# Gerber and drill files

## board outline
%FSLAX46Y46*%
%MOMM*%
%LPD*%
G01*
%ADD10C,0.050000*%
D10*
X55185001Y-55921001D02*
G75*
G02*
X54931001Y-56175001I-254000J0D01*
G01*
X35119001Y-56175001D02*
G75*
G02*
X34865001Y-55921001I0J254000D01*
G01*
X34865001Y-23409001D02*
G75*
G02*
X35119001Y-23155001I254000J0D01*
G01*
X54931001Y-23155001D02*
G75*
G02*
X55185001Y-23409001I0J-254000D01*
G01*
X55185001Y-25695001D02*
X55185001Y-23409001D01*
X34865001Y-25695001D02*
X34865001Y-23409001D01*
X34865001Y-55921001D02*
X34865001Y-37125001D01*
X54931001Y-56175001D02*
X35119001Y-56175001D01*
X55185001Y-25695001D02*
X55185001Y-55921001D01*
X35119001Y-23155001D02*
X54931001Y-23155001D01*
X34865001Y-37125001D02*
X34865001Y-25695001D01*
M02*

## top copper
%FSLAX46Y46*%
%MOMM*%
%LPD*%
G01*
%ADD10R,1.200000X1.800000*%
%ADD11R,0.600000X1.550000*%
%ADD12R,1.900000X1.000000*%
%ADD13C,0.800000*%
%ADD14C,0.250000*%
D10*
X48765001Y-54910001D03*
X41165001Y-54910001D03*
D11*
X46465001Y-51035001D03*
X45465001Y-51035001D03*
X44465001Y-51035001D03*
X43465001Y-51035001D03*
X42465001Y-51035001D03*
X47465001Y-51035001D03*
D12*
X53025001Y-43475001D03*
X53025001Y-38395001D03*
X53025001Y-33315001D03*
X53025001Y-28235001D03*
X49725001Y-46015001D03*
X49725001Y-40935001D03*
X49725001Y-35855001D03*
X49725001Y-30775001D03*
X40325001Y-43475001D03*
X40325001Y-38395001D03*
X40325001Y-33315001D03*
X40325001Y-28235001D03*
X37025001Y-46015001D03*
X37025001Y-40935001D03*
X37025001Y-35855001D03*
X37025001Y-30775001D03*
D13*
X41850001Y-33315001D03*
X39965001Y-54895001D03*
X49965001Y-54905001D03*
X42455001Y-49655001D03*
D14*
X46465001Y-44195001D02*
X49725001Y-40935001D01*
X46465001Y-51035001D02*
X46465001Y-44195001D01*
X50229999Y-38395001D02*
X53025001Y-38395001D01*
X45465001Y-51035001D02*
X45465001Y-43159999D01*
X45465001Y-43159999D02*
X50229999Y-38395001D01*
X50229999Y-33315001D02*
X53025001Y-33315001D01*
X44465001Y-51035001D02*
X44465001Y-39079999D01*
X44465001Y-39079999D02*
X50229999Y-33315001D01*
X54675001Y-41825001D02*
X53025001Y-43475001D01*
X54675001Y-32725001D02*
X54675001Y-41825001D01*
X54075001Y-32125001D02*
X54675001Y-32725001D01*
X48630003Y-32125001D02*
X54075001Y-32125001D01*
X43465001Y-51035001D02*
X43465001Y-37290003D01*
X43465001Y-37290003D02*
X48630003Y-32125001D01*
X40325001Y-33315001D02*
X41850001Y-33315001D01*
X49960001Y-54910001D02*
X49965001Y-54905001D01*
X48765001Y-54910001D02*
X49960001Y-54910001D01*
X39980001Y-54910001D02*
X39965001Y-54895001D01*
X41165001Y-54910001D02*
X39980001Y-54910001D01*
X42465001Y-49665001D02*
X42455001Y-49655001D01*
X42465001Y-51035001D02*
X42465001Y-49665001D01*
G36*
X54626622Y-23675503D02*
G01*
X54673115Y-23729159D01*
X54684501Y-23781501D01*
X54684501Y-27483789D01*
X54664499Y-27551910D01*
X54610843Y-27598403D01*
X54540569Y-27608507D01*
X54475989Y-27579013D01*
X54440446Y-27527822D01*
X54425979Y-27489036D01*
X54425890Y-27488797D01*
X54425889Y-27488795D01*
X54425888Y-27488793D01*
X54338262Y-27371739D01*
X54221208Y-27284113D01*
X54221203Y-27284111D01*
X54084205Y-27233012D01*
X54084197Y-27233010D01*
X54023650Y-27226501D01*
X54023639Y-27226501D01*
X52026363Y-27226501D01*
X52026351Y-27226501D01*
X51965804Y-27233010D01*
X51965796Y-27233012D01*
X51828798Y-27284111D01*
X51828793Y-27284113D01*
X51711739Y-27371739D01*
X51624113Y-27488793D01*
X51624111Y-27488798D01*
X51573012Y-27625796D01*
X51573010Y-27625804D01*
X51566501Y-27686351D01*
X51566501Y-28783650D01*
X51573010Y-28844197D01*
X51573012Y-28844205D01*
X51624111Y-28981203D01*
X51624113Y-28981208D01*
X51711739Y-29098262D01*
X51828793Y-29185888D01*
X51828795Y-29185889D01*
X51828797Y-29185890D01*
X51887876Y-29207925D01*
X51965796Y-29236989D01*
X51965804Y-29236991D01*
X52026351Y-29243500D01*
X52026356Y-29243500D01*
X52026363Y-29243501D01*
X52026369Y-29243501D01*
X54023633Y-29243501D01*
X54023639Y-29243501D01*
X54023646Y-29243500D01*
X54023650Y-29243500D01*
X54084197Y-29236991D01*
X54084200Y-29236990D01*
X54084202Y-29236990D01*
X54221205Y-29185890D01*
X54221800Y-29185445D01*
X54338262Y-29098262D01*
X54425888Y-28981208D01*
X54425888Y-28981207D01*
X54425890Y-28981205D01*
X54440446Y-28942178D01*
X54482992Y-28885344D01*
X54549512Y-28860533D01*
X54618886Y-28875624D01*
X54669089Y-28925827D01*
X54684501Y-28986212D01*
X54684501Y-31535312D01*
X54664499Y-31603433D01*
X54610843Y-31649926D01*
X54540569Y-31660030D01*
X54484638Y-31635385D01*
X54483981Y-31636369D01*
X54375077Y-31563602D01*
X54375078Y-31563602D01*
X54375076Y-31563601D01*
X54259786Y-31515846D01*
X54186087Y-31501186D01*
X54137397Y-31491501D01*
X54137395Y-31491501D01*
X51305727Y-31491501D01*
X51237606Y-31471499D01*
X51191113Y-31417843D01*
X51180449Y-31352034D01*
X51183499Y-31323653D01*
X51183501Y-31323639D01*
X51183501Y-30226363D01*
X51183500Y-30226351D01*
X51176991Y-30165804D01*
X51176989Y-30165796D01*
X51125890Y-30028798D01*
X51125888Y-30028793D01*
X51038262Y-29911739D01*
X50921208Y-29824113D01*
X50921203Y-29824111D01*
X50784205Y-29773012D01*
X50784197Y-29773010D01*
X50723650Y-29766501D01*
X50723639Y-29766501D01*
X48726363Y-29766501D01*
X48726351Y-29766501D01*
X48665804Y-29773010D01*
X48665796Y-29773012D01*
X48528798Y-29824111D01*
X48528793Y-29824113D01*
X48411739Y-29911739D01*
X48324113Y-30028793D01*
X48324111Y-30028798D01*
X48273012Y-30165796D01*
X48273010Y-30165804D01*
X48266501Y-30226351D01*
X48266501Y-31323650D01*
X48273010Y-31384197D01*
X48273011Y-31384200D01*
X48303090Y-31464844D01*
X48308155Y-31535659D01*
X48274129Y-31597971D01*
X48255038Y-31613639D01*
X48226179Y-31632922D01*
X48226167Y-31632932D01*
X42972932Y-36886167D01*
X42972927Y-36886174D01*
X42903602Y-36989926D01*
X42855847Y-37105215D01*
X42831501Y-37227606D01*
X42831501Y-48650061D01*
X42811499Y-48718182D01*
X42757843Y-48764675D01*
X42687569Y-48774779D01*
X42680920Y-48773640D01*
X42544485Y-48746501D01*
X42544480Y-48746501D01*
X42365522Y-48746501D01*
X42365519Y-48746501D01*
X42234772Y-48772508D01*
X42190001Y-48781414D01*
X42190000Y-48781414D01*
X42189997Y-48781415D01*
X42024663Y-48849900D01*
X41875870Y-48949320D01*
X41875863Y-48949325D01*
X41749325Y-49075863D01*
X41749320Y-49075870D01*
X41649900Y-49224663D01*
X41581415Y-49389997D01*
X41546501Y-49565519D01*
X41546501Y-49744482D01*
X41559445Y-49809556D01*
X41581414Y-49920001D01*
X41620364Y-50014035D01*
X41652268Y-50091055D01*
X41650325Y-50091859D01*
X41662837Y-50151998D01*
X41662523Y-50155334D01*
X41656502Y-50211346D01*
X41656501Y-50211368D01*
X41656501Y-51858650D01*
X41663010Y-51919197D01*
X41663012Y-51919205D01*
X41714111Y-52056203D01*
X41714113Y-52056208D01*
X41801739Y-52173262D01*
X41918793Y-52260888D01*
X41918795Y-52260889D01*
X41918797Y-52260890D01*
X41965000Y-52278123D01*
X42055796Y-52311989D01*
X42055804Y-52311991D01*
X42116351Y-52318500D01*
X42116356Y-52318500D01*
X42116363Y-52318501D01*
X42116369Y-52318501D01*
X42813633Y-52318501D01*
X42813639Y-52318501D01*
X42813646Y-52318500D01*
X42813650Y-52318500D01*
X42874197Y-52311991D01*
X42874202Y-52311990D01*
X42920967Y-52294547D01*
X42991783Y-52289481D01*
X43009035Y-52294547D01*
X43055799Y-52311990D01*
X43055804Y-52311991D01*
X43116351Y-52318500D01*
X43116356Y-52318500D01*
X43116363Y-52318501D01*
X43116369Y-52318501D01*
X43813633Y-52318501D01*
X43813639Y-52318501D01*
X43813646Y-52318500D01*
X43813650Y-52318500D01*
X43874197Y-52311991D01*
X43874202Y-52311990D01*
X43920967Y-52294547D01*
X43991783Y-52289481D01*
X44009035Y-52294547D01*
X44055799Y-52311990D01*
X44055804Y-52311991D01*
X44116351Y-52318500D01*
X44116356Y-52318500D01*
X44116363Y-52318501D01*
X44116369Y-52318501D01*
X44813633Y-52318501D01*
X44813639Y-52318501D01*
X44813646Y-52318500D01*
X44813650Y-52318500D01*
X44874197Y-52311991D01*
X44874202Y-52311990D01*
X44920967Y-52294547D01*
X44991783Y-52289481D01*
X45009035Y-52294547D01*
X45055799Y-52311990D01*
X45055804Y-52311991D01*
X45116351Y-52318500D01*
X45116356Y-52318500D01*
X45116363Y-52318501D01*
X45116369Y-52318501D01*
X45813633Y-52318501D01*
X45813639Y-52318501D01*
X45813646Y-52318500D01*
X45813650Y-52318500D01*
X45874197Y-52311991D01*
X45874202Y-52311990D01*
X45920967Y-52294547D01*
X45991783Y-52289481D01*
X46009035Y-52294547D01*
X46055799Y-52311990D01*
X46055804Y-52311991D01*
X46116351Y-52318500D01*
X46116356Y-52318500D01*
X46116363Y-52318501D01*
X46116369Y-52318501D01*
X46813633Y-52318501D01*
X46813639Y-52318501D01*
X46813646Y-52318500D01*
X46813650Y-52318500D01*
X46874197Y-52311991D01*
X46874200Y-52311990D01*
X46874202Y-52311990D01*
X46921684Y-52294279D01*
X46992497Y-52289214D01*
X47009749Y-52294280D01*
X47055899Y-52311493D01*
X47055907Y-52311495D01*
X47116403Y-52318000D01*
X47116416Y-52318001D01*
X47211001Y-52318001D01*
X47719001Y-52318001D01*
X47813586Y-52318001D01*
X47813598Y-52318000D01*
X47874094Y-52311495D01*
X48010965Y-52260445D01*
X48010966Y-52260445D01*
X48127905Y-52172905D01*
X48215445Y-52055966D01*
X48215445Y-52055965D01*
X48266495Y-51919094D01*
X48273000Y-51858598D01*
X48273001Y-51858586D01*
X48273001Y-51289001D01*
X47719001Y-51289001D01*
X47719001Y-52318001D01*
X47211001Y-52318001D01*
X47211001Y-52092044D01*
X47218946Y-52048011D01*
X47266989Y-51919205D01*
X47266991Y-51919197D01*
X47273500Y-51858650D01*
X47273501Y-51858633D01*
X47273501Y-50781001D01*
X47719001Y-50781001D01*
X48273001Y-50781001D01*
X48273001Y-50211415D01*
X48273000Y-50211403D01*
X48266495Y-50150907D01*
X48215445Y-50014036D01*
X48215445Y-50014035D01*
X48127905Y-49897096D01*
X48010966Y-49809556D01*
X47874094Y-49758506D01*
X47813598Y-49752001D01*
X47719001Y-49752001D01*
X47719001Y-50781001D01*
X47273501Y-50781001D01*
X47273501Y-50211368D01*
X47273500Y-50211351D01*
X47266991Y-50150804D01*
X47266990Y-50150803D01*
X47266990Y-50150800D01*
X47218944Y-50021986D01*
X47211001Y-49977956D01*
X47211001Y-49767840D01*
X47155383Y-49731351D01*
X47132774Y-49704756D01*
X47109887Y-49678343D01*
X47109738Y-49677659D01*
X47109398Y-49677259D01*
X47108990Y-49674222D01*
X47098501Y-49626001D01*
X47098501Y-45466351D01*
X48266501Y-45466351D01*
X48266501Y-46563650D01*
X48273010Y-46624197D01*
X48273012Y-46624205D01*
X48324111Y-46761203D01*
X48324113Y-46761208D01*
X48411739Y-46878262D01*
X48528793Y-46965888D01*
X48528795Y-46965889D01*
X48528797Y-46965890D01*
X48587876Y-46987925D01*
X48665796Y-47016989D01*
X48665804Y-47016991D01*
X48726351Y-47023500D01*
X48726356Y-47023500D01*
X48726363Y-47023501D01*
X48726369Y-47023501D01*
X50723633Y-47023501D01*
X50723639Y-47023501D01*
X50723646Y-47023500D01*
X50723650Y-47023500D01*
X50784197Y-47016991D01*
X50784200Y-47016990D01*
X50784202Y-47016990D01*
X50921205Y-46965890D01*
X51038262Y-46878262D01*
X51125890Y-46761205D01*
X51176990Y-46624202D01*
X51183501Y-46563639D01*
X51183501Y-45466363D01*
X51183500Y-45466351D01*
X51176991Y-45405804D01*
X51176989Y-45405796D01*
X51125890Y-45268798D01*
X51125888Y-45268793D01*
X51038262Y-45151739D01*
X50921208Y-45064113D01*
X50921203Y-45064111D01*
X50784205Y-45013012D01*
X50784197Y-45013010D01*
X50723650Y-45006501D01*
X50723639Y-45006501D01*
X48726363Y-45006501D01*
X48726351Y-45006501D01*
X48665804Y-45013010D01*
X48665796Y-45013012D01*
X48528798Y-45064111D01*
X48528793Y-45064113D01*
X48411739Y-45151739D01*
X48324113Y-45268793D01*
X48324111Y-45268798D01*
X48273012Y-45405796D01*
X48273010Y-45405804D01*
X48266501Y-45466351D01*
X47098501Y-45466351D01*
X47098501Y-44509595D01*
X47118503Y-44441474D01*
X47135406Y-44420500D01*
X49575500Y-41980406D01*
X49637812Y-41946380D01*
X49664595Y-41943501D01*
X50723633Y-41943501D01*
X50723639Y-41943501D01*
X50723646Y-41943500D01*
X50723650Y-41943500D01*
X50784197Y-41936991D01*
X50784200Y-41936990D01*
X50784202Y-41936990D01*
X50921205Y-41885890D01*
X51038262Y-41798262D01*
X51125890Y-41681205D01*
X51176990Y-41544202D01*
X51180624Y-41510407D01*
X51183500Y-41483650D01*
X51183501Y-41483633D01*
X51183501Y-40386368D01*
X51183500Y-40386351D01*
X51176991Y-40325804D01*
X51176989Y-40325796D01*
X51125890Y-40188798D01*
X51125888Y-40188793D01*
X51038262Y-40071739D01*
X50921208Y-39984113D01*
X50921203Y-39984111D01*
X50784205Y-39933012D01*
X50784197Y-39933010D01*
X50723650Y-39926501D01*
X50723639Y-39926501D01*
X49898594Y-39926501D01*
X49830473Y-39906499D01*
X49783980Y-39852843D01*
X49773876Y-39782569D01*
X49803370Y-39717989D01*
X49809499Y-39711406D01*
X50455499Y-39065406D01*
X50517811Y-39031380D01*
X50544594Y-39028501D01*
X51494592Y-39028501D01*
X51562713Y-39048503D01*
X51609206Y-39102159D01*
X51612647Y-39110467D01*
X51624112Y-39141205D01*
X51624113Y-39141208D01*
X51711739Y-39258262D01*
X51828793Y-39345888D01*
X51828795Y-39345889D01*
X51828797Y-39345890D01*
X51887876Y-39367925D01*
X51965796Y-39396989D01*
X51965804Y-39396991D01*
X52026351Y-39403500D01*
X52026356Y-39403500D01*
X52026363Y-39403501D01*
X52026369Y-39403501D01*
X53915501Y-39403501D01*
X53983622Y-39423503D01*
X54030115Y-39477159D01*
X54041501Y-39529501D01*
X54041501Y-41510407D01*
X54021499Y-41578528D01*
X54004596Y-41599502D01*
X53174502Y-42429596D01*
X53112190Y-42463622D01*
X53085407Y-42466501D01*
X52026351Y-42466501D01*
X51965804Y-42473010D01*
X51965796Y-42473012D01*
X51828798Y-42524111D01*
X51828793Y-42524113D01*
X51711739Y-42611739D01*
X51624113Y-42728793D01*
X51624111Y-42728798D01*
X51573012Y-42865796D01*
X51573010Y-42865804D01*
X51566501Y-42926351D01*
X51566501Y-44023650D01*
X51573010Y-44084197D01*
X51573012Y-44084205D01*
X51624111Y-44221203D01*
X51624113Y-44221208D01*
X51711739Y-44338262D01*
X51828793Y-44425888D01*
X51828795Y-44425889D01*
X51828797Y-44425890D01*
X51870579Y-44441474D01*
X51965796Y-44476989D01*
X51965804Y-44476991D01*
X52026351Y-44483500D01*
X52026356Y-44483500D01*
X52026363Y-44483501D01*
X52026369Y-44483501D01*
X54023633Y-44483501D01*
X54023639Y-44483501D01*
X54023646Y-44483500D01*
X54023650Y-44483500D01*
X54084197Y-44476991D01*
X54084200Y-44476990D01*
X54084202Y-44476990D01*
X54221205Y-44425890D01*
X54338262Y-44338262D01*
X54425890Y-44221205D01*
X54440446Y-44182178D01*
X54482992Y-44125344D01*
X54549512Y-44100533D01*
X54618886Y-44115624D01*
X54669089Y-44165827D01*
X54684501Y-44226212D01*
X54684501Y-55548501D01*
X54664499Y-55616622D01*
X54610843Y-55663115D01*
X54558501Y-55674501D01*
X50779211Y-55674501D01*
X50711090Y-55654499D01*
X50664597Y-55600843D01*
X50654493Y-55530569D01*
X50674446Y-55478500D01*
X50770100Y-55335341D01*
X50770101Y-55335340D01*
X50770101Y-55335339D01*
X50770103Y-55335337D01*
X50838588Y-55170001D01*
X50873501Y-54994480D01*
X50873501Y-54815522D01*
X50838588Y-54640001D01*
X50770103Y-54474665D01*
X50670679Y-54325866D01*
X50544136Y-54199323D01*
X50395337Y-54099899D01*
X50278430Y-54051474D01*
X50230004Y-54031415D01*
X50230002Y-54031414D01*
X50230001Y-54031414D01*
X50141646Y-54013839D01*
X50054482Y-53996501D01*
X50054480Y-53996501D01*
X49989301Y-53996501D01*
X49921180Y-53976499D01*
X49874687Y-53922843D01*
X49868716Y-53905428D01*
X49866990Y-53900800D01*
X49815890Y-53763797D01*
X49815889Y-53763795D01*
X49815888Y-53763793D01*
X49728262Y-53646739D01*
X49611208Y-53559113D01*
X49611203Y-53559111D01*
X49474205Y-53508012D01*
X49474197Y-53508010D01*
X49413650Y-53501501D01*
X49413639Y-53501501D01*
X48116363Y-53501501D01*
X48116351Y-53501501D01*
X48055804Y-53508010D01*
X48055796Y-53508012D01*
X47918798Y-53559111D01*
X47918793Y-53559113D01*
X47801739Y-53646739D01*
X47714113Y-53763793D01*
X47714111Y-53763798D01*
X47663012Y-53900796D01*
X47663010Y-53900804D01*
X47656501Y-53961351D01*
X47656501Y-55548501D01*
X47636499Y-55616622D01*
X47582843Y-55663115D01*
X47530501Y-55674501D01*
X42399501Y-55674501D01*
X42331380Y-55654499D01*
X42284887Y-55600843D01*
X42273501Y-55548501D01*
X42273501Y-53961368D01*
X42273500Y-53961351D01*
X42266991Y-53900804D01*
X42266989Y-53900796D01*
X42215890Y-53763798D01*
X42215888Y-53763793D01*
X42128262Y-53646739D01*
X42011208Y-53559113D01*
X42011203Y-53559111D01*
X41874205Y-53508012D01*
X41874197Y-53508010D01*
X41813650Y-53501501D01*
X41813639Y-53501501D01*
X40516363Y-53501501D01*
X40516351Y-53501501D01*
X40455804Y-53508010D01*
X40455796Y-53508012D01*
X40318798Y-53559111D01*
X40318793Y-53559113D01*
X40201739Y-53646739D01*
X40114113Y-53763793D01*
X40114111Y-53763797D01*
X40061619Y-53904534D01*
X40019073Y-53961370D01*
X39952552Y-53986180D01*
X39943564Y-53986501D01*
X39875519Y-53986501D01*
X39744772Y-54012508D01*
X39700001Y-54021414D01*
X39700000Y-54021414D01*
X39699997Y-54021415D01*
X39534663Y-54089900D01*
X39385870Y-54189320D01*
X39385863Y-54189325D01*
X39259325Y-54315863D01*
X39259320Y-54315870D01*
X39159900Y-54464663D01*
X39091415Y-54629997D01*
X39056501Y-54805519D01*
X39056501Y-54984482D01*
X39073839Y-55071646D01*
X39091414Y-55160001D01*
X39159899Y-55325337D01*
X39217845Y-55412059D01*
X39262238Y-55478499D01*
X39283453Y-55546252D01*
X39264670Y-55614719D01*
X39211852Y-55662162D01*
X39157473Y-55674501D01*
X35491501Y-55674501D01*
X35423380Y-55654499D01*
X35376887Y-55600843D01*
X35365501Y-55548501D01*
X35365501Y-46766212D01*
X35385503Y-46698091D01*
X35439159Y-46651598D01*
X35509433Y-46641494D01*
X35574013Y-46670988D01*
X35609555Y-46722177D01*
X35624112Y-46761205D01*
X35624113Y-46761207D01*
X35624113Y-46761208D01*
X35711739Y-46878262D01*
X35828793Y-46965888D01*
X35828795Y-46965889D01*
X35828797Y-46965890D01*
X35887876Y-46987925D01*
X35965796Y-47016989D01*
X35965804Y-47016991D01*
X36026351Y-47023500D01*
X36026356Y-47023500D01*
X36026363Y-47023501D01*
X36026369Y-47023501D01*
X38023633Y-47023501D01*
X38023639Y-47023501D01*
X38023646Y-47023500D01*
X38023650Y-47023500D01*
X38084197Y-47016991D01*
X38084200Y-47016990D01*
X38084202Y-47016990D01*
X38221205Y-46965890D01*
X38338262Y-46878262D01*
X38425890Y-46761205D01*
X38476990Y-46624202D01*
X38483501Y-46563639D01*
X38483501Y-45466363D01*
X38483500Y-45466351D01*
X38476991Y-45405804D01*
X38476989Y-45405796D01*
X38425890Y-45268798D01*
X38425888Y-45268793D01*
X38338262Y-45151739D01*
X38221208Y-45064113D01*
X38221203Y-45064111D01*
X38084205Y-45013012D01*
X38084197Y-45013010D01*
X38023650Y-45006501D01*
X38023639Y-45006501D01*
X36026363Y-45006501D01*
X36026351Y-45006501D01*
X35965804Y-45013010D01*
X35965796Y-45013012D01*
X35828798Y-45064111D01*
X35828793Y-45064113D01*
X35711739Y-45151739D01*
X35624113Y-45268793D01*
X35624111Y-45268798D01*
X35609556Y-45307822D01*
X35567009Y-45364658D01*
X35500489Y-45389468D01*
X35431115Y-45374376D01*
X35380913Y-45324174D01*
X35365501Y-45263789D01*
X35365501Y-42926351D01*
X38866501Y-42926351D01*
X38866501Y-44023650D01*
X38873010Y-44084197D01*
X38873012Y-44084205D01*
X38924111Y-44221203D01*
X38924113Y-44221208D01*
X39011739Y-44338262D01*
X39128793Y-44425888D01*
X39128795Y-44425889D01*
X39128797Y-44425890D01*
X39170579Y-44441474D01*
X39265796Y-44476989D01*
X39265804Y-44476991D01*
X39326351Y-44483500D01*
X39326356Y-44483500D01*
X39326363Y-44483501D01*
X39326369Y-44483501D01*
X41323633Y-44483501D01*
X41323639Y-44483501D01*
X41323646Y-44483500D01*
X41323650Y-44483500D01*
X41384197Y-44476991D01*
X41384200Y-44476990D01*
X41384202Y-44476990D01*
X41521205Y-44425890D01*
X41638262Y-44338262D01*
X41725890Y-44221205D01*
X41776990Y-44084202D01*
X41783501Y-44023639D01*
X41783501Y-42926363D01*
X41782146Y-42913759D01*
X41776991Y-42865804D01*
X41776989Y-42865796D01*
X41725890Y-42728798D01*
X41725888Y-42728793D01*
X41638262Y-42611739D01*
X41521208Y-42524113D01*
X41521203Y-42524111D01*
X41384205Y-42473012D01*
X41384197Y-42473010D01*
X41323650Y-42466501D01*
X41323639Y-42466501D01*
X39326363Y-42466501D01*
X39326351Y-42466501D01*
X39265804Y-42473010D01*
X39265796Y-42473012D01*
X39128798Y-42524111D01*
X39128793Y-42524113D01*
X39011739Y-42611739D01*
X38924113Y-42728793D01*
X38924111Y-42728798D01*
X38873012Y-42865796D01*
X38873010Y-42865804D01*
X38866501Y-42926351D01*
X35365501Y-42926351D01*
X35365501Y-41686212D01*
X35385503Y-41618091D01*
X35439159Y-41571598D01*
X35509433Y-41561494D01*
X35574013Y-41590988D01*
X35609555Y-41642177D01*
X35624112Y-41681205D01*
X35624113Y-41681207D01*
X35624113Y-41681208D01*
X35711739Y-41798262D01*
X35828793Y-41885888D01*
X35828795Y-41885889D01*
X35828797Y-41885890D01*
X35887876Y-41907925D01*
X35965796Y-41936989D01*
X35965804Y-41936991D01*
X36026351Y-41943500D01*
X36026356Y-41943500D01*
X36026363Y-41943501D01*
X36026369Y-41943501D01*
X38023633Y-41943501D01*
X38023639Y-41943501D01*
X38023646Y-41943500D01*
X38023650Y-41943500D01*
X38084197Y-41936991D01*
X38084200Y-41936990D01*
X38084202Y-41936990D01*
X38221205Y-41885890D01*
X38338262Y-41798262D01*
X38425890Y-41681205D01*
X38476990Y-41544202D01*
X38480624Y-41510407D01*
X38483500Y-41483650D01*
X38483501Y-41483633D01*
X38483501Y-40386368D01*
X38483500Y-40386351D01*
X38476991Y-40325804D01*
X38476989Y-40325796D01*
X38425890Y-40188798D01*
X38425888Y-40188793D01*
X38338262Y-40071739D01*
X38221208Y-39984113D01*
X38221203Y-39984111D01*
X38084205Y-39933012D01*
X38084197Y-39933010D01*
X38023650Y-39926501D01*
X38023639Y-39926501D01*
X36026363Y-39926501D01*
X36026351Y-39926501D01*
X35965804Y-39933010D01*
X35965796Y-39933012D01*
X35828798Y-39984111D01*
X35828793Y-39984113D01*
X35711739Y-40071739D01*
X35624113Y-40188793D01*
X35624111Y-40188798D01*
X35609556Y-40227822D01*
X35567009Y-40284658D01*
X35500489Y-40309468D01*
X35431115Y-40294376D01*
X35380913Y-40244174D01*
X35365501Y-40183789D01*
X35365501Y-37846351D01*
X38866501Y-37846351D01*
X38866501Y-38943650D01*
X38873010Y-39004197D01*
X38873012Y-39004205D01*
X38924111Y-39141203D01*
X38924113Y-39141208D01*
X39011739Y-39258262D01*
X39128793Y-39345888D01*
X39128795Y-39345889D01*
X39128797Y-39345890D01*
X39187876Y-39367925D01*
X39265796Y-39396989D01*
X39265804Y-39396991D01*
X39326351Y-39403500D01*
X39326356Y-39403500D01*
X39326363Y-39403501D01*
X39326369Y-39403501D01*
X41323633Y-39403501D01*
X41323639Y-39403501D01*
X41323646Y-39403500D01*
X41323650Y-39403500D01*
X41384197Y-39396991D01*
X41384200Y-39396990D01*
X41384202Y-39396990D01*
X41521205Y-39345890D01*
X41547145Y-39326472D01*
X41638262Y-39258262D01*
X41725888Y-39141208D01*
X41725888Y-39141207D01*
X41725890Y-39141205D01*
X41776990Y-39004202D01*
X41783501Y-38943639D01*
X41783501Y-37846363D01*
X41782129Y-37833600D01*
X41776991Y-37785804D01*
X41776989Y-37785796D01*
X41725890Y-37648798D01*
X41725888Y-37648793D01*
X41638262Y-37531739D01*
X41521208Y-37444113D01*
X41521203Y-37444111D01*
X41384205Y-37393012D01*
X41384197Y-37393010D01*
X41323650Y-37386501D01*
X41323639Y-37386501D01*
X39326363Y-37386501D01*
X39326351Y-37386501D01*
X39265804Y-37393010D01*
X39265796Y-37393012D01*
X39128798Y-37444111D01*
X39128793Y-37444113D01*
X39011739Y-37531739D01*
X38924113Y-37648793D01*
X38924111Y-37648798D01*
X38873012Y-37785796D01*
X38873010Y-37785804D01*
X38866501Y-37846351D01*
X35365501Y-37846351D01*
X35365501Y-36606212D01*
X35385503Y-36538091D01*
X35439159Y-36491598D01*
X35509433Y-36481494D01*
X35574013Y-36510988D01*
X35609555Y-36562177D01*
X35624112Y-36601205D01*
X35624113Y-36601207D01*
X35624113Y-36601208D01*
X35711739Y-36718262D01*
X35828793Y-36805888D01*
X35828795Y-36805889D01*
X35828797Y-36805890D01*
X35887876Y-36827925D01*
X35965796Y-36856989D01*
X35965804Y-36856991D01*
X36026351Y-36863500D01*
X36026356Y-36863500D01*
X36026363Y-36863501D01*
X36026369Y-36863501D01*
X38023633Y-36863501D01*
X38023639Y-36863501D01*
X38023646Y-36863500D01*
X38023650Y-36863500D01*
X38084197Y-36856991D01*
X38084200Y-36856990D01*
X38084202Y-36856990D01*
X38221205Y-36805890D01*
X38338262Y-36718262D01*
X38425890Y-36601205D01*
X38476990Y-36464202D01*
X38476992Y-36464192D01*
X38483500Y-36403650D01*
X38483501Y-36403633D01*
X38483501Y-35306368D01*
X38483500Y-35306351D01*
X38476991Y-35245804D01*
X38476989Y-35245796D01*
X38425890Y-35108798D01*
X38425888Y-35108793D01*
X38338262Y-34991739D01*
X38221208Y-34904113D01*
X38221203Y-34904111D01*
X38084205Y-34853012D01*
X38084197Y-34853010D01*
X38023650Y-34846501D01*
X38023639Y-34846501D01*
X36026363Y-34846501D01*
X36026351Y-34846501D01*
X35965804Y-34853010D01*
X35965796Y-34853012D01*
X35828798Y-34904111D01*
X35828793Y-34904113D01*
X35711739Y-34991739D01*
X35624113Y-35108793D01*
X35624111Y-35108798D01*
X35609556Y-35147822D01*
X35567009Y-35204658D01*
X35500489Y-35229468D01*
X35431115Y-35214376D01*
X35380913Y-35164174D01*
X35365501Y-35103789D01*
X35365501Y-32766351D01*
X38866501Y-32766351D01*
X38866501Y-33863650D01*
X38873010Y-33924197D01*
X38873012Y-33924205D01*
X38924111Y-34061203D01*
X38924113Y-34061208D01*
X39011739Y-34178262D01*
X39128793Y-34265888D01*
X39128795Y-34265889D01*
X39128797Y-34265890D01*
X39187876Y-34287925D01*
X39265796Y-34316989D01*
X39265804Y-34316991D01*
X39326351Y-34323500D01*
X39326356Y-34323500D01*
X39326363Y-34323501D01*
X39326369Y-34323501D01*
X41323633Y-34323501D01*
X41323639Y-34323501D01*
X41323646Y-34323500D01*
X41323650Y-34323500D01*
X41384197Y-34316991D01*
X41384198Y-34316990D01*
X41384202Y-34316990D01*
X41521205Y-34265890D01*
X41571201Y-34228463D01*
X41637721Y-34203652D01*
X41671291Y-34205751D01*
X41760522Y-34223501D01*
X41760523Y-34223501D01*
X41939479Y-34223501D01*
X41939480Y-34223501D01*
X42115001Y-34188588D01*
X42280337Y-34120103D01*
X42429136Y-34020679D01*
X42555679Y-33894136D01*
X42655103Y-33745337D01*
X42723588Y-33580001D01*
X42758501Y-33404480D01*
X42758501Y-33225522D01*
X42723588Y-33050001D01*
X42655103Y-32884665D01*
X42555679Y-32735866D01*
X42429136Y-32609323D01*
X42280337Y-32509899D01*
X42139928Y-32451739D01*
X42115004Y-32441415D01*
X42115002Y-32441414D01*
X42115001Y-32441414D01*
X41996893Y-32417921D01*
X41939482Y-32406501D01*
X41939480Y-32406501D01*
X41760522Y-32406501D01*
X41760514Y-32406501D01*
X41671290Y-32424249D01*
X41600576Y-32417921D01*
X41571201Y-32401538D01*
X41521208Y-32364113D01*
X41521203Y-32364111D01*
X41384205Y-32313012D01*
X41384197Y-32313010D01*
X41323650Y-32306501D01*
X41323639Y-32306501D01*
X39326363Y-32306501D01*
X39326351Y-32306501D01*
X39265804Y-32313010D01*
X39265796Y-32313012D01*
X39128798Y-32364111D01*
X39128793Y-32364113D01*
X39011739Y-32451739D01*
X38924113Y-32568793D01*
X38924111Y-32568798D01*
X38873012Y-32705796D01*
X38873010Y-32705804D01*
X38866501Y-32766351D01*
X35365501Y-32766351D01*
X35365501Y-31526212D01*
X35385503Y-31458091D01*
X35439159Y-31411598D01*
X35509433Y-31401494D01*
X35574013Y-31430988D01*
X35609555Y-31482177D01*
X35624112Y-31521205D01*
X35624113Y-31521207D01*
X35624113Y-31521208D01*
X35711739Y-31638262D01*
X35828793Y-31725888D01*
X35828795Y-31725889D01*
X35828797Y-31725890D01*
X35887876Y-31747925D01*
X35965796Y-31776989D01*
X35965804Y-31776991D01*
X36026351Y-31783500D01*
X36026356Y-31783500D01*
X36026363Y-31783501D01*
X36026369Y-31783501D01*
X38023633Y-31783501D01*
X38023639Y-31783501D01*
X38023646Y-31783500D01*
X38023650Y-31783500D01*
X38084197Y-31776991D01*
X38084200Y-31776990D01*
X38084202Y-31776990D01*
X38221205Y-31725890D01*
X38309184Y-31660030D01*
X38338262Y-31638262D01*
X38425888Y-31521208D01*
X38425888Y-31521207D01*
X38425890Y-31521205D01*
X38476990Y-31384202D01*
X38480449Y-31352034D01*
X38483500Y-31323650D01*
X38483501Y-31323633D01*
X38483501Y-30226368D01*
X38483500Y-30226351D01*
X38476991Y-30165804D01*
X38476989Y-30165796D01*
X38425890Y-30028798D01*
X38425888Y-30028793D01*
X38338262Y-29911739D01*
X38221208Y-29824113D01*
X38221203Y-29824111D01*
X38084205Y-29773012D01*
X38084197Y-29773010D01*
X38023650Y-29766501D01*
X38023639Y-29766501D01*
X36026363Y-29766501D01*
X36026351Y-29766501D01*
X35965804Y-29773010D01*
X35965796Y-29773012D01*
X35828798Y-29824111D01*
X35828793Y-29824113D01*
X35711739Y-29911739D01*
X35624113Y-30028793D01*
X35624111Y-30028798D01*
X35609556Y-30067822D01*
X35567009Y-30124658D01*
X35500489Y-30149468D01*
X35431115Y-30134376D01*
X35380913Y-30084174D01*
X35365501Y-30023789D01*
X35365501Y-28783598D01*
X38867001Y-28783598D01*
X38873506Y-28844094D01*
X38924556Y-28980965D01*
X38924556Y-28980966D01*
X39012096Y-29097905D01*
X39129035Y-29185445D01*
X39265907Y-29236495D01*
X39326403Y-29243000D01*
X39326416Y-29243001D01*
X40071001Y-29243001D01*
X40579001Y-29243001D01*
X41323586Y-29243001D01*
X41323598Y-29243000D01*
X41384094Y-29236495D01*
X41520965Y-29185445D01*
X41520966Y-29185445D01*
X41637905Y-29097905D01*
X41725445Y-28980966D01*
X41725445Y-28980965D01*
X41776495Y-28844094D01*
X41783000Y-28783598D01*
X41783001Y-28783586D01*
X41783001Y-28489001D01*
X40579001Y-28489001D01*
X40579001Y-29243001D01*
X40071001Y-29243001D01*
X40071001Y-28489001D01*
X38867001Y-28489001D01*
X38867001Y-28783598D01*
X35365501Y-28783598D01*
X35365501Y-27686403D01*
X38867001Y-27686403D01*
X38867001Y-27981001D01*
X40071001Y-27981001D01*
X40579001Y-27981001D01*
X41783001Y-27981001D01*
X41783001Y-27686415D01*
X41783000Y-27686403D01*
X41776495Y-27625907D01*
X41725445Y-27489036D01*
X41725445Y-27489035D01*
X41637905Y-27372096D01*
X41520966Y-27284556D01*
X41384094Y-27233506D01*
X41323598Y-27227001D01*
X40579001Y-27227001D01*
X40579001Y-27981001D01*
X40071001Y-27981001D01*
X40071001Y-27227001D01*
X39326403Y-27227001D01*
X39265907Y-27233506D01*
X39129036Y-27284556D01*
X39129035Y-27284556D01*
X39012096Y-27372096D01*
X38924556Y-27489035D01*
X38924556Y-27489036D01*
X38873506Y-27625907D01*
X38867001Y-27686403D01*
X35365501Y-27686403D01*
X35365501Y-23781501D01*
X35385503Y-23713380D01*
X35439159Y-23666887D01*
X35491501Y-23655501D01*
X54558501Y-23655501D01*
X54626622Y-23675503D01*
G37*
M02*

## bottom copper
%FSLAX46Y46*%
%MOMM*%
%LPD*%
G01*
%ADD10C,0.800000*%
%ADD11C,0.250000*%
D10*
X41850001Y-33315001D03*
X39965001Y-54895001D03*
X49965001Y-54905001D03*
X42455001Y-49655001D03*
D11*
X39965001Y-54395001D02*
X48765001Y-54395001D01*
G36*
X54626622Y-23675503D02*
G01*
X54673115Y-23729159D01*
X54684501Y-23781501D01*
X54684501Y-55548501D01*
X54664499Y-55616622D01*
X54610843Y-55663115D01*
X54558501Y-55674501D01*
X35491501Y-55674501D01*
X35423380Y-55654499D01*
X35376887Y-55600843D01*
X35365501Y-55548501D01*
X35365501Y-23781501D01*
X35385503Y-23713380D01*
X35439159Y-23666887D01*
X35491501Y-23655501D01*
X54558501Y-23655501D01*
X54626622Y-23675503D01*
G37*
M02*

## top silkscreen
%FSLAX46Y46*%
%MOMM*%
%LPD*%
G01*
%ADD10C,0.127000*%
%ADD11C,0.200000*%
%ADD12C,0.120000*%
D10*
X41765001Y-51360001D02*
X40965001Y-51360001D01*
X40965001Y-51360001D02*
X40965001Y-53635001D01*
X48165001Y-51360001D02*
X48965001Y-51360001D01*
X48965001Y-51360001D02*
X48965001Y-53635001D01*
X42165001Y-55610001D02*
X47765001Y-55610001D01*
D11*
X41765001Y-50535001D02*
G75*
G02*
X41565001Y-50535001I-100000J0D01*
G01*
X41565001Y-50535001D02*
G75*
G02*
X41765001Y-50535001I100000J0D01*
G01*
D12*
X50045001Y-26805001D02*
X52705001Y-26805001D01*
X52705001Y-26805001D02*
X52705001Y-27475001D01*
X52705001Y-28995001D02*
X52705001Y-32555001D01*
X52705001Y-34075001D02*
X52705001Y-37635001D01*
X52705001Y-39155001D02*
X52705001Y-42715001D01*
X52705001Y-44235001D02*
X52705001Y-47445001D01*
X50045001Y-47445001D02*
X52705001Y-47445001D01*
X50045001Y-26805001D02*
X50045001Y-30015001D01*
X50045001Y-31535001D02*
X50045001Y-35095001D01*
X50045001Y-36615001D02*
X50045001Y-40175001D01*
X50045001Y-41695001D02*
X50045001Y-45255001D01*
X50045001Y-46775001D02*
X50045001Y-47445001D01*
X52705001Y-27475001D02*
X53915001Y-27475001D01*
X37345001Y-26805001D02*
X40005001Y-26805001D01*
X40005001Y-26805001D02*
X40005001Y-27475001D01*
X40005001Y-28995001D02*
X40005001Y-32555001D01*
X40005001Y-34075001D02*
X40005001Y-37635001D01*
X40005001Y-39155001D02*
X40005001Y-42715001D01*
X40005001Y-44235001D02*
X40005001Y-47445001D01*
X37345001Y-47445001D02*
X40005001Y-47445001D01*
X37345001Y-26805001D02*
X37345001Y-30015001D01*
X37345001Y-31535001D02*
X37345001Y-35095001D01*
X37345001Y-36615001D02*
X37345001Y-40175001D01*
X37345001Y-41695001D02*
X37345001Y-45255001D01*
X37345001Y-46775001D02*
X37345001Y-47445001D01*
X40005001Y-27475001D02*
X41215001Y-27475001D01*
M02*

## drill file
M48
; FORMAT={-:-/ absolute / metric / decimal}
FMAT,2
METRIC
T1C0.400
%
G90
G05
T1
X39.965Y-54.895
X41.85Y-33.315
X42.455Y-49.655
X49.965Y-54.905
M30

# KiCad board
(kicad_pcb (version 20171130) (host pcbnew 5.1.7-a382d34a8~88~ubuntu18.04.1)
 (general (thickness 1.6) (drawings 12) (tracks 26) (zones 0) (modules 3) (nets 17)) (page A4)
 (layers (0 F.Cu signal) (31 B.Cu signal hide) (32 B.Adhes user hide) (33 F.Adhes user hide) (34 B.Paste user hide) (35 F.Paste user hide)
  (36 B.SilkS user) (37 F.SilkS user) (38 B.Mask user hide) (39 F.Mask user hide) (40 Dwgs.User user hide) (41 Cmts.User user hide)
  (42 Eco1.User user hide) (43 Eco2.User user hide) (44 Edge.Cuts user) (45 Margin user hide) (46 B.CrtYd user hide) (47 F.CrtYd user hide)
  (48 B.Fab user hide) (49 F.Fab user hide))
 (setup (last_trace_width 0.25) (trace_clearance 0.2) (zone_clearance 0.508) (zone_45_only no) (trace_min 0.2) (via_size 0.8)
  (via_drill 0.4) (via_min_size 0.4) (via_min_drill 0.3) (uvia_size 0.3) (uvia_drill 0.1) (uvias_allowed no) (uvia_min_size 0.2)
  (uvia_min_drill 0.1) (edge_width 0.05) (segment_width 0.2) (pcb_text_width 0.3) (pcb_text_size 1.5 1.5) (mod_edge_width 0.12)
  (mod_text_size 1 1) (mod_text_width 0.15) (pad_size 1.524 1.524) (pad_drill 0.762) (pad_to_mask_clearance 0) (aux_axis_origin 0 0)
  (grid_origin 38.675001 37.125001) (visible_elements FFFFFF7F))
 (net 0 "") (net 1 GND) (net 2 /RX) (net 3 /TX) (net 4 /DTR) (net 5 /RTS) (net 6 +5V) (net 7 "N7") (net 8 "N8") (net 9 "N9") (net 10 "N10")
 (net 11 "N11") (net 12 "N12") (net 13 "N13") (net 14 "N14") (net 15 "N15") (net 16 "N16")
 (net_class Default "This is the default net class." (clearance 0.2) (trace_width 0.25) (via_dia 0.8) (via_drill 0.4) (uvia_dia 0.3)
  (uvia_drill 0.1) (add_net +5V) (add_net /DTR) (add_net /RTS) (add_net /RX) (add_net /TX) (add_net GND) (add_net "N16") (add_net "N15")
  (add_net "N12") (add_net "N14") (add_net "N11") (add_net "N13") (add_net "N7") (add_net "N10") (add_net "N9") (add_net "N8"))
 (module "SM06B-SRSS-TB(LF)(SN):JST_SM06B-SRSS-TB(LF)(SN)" (layer F.Cu) (at 44.965001 51.035001)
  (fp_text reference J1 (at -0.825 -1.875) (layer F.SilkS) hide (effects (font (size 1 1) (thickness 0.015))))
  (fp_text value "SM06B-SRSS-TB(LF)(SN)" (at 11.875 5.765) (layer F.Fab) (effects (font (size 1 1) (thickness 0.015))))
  (fp_line (start -3.2 0.325) (end -4 0.325) (layer F.SilkS) (width 0.127))
  (fp_line (start -4 0.325) (end -4 2.6) (layer F.SilkS) (width 0.127))
  (fp_line (start 3.2 0.325) (end 4 0.325) (layer F.SilkS) (width 0.127))
  (fp_line (start 4 0.325) (end 4 2.6) (layer F.SilkS) (width 0.127))
  (fp_line (start -2.8 4.575) (end 2.8 4.575) (layer F.SilkS) (width 0.127))
  (fp_circle (center -3.3 -0.5) (end -3.2 -0.5) (layer F.SilkS) (width 0.2))
  (pad S2 smd rect (at 3.8 3.875) (size 1.2 1.8) (layers F.Cu F.Paste F.Mask) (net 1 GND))
  (pad S1 smd rect (at -3.8 3.875) (size 1.2 1.8) (layers F.Cu F.Paste F.Mask) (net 1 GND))
  (pad 5 smd rect (at 1.5 0) (size 0.6 1.55) (layers F.Cu F.Paste F.Mask) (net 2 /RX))
  (pad 4 smd rect (at 0.5 0) (size 0.6 1.55) (layers F.Cu F.Paste F.Mask) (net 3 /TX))
  (pad 3 smd rect (at -0.5 0) (size 0.6 1.55) (layers F.Cu F.Paste F.Mask) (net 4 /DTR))
  (pad 2 smd rect (at -1.5 0) (size 0.6 1.55) (layers F.Cu F.Paste F.Mask) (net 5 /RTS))
  (pad 1 smd rect (at -2.5 0) (size 0.6 1.55) (layers F.Cu F.Paste F.Mask) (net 1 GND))
  (pad 6 smd rect (at 2.5 0) (size 0.6 1.55) (layers F.Cu F.Paste F.Mask) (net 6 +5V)))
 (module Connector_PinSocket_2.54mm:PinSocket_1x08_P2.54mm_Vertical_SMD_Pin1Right (layer F.Cu) (at 51.375001 37.125001)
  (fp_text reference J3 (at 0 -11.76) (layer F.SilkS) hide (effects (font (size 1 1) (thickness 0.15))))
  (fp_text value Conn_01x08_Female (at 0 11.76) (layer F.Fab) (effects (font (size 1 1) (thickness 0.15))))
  (fp_line (start -1.33 -10.32) (end 1.33 -10.32) (layer F.SilkS) (width 0.12))
  (fp_line (start 1.33 -10.32) (end 1.33 -9.65) (layer F.SilkS) (width 0.12))
  (fp_line (start 1.33 -8.13) (end 1.33 -4.57) (layer F.SilkS) (width 0.12))
  (fp_line (start 1.33 -3.05) (end 1.33 0.51) (layer F.SilkS) (width 0.12))
  (fp_line (start 1.33 2.03) (end 1.33 5.59) (layer F.SilkS) (width 0.12))
  (fp_line (start 1.33 7.11) (end 1.33 10.32) (layer F.SilkS) (width 0.12))
  (fp_line (start -1.33 10.32) (end 1.33 10.32) (layer F.SilkS) (width 0.12))
  (fp_line (start -1.33 -10.32) (end -1.33 -7.11) (layer F.SilkS) (width 0.12))
  (fp_line (start -1.33 -5.59) (end -1.33 -2.03) (layer F.SilkS) (width 0.12))
  (fp_line (start -1.33 -0.51) (end -1.33 3.05) (layer F.SilkS) (width 0.12))
  (fp_line (start -1.33 4.57) (end -1.33 8.13) (layer F.SilkS) (width 0.12))
  (fp_line (start -1.33 9.65) (end -1.33 10.32) (layer F.SilkS) (width 0.12))
  (fp_line (start 1.33 -9.65) (end 2.54 -9.65) (layer F.SilkS) (width 0.12))
  (pad 7 smd rect (at 1.65 6.35) (size 1.9 1) (layers F.Cu F.Paste F.Mask) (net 5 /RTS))
  (pad 5 smd rect (at 1.65 1.27) (size 1.9 1) (layers F.Cu F.Paste F.Mask) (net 3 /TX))
  (pad 3 smd rect (at 1.65 -3.81) (size 1.9 1) (layers F.Cu F.Paste F.Mask) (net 4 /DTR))
  (pad 1 smd rect (at 1.65 -8.89) (size 1.9 1) (layers F.Cu F.Paste F.Mask) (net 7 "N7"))
  (pad 8 smd rect (at -1.65 8.89) (size 1.9 1) (layers F.Cu F.Paste F.Mask) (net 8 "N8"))
  (pad 6 smd rect (at -1.65 3.81) (size 1.9 1) (layers F.Cu F.Paste F.Mask) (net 2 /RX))
  (pad 4 smd rect (at -1.65 -1.27) (size 1.9 1) (layers F.Cu F.Paste F.Mask) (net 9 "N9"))
  (pad 2 smd rect (at -1.65 -6.35) (size 1.9 1) (layers F.Cu F.Paste F.Mask) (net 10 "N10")))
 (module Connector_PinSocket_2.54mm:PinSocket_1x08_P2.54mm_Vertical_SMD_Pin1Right (layer F.Cu) (at 38.675001 37.125001)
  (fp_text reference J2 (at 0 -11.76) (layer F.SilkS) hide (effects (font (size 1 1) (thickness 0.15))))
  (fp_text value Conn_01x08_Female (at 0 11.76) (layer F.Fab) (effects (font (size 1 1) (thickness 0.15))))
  (fp_line (start -1.33 -10.32) (end 1.33 -10.32) (layer F.SilkS) (width 0.12))
  (fp_line (start 1.33 -10.32) (end 1.33 -9.65) (layer F.SilkS) (width 0.12))
  (fp_line (start 1.33 -8.13) (end 1.33 -4.57) (layer F.SilkS) (width 0.12))
  (fp_line (start 1.33 -3.05) (end 1.33 0.51) (layer F.SilkS) (width 0.12))
  (fp_line (start 1.33 2.03) (end 1.33 5.59) (layer F.SilkS) (width 0.12))
  (fp_line (start 1.33 7.11) (end 1.33 10.32) (layer F.SilkS) (width 0.12))
  (fp_line (start -1.33 10.32) (end 1.33 10.32) (layer F.SilkS) (width 0.12))
  (fp_line (start -1.33 -10.32) (end -1.33 -7.11) (layer F.SilkS) (width 0.12))
  (fp_line (start -1.33 -5.59) (end -1.33 -2.03) (layer F.SilkS) (width 0.12))
  (fp_line (start -1.33 -0.51) (end -1.33 3.05) (layer F.SilkS) (width 0.12))
  (fp_line (start -1.33 4.57) (end -1.33 8.13) (layer F.SilkS) (width 0.12))
  (fp_line (start -1.33 9.65) (end -1.33 10.32) (layer F.SilkS) (width 0.12))
  (fp_line (start 1.33 -9.65) (end 2.54 -9.65) (layer F.SilkS) (width 0.12))
  (pad 7 smd rect (at 1.65 6.35) (size 1.9 1) (layers F.Cu F.Paste F.Mask) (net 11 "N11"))
  (pad 5 smd rect (at 1.65 1.27) (size 1.9 1) (layers F.Cu F.Paste F.Mask) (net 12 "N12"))
  (pad 3 smd rect (at 1.65 -3.81) (size 1.9 1) (layers F.Cu F.Paste F.Mask) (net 1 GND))
  (pad 1 smd rect (at 1.65 -8.89) (size 1.9 1) (layers F.Cu F.Paste F.Mask) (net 6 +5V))
  (pad 8 smd rect (at -1.65 8.89) (size 1.9 1) (layers F.Cu F.Paste F.Mask) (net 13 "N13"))
  (pad 6 smd rect (at -1.65 3.81) (size 1.9 1) (layers F.Cu F.Paste F.Mask) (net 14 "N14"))
  (pad 4 smd rect (at -1.65 -1.27) (size 1.9 1) (layers F.Cu F.Paste F.Mask) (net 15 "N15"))
  (pad 2 smd rect (at -1.65 -6.35) (size 1.9 1) (layers F.Cu F.Paste F.Mask) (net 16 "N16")))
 (gr_arc (start 54.931001 55.921001) (end 54.931001 56.175001) (angle -90) (layer Edge.Cuts) (width 0.05))
 (gr_arc (start 35.119001 55.921001) (end 34.865001 55.921001) (angle -90) (layer Edge.Cuts) (width 0.05))
 (gr_arc (start 35.119001 23.409001) (end 35.119001 23.155001) (angle -90) (layer Edge.Cuts) (width 0.05))
 (gr_arc (start 54.931001 23.409001) (end 55.185001 23.409001) (angle -90) (layer Edge.Cuts) (width 0.05))
 (gr_line (start 55.185001 25.695001) (end 55.185001 23.409001) (layer Edge.Cuts) (width 0.05))
 (gr_line (start 34.865001 25.695001) (end 34.865001 23.409001) (layer Edge.Cuts) (width 0.05))
 (gr_line (start 34.865001 55.921001) (end 34.865001 37.125001) (layer Edge.Cuts) (width 0.05))
 (gr_line (start 54.931001 56.175001) (end 35.119001 56.175001) (layer Edge.Cuts) (width 0.05))
 (gr_line (start 55.185001 25.695001) (end 55.185001 55.921001) (layer Edge.Cuts) (width 0.05))
 (gr_line (start 35.119001 23.155001) (end 54.931001 23.155001) (layer Edge.Cuts) (width 0.05))
 (gr_line (start 34.865001 37.125001) (end 34.865001 25.695001) (layer Edge.Cuts) (width 0.05))
 (segment (start 46.465001 44.195001) (end 49.725001 40.935001) (width 0.25) (layer F.Cu) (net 2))
 (segment (start 46.465001 51.035001) (end 46.465001 44.195001) (width 0.25) (layer F.Cu) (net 2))
 (segment (start 50.229999 38.395001) (end 53.025001 38.395001) (width 0.25) (layer F.Cu) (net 3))
 (segment (start 45.465001 51.035001) (end 45.465001 43.159999) (width 0.25) (layer F.Cu) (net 3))
 (segment (start 45.465001 43.159999) (end 50.229999 38.395001) (width 0.25) (layer F.Cu) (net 3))
 (segment (start 50.229999 33.315001) (end 53.025001 33.315001) (width 0.25) (layer F.Cu) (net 4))
 (segment (start 44.465001 51.035001) (end 44.465001 39.079999) (width 0.25) (layer F.Cu) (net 4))
 (segment (start 44.465001 39.079999) (end 50.229999 33.315001) (width 0.25) (layer F.Cu) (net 4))
 (segment (start 54.675001 41.825001) (end 53.025001 43.475001) (width 0.25) (layer F.Cu) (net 5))
 (segment (start 54.675001 32.725001) (end 54.675001 41.825001) (width 0.25) (layer F.Cu) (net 5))
 (segment (start 54.075001 32.125001) (end 54.675001 32.725001) (width 0.25) (layer F.Cu) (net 5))
 (segment (start 48.630003 32.125001) (end 54.075001 32.125001) (width 0.25) (layer F.Cu) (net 5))
 (segment (start 43.465001 51.035001) (end 43.465001 37.290003) (width 0.25) (layer F.Cu) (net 5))
 (segment (start 43.465001 37.290003) (end 48.630003 32.125001) (width 0.25) (layer F.Cu) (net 5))
 (via (at 41.850001 33.315001) (size 0.8) (drill 0.4) (layers F.Cu B.Cu) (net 1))
 (segment (start 40.325001 33.315001) (end 41.850001 33.315001) (width 0.25) (layer F.Cu) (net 1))
 (via (at 39.965001 54.895001) (size 0.8) (drill 0.4) (layers F.Cu B.Cu) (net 1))
 (segment (start 39.965001 54.395001) (end 48.765001 54.395001) (width 0.25) (layer B.Cu) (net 1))
 (via (at 49.965001 54.905001) (size 0.8) (drill 0.4) (layers F.Cu B.Cu) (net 1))
 (via (at 42.455001 49.655001) (size 0.8) (drill 0.4) (layers F.Cu B.Cu) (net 1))
 (segment (start 49.960001 54.910001) (end 49.965001 54.905001) (width 0.25) (layer F.Cu) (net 1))
 (segment (start 48.765001 54.910001) (end 49.960001 54.910001) (width 0.25) (layer F.Cu) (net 1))
 (segment (start 39.980001 54.910001) (end 39.965001 54.895001) (width 0.25) (layer F.Cu) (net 1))
 (segment (start 41.165001 54.910001) (end 39.980001 54.910001) (width 0.25) (layer F.Cu) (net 1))
 (segment (start 42.465001 49.665001) (end 42.455001 49.655001) (width 0.25) (layer F.Cu) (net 1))
 (segment (start 42.465001 51.035001) (end 42.465001 49.665001) (width 0.25) (layer F.Cu) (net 1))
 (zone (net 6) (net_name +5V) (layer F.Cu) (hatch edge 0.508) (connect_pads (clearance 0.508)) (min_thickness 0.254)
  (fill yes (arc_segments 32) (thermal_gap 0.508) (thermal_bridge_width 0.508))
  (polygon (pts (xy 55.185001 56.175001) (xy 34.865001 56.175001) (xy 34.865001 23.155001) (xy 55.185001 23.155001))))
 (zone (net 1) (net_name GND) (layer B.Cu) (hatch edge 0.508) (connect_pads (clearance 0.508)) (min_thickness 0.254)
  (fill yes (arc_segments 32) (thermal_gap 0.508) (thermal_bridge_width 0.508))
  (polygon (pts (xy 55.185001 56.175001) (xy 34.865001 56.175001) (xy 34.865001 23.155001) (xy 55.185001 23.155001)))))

